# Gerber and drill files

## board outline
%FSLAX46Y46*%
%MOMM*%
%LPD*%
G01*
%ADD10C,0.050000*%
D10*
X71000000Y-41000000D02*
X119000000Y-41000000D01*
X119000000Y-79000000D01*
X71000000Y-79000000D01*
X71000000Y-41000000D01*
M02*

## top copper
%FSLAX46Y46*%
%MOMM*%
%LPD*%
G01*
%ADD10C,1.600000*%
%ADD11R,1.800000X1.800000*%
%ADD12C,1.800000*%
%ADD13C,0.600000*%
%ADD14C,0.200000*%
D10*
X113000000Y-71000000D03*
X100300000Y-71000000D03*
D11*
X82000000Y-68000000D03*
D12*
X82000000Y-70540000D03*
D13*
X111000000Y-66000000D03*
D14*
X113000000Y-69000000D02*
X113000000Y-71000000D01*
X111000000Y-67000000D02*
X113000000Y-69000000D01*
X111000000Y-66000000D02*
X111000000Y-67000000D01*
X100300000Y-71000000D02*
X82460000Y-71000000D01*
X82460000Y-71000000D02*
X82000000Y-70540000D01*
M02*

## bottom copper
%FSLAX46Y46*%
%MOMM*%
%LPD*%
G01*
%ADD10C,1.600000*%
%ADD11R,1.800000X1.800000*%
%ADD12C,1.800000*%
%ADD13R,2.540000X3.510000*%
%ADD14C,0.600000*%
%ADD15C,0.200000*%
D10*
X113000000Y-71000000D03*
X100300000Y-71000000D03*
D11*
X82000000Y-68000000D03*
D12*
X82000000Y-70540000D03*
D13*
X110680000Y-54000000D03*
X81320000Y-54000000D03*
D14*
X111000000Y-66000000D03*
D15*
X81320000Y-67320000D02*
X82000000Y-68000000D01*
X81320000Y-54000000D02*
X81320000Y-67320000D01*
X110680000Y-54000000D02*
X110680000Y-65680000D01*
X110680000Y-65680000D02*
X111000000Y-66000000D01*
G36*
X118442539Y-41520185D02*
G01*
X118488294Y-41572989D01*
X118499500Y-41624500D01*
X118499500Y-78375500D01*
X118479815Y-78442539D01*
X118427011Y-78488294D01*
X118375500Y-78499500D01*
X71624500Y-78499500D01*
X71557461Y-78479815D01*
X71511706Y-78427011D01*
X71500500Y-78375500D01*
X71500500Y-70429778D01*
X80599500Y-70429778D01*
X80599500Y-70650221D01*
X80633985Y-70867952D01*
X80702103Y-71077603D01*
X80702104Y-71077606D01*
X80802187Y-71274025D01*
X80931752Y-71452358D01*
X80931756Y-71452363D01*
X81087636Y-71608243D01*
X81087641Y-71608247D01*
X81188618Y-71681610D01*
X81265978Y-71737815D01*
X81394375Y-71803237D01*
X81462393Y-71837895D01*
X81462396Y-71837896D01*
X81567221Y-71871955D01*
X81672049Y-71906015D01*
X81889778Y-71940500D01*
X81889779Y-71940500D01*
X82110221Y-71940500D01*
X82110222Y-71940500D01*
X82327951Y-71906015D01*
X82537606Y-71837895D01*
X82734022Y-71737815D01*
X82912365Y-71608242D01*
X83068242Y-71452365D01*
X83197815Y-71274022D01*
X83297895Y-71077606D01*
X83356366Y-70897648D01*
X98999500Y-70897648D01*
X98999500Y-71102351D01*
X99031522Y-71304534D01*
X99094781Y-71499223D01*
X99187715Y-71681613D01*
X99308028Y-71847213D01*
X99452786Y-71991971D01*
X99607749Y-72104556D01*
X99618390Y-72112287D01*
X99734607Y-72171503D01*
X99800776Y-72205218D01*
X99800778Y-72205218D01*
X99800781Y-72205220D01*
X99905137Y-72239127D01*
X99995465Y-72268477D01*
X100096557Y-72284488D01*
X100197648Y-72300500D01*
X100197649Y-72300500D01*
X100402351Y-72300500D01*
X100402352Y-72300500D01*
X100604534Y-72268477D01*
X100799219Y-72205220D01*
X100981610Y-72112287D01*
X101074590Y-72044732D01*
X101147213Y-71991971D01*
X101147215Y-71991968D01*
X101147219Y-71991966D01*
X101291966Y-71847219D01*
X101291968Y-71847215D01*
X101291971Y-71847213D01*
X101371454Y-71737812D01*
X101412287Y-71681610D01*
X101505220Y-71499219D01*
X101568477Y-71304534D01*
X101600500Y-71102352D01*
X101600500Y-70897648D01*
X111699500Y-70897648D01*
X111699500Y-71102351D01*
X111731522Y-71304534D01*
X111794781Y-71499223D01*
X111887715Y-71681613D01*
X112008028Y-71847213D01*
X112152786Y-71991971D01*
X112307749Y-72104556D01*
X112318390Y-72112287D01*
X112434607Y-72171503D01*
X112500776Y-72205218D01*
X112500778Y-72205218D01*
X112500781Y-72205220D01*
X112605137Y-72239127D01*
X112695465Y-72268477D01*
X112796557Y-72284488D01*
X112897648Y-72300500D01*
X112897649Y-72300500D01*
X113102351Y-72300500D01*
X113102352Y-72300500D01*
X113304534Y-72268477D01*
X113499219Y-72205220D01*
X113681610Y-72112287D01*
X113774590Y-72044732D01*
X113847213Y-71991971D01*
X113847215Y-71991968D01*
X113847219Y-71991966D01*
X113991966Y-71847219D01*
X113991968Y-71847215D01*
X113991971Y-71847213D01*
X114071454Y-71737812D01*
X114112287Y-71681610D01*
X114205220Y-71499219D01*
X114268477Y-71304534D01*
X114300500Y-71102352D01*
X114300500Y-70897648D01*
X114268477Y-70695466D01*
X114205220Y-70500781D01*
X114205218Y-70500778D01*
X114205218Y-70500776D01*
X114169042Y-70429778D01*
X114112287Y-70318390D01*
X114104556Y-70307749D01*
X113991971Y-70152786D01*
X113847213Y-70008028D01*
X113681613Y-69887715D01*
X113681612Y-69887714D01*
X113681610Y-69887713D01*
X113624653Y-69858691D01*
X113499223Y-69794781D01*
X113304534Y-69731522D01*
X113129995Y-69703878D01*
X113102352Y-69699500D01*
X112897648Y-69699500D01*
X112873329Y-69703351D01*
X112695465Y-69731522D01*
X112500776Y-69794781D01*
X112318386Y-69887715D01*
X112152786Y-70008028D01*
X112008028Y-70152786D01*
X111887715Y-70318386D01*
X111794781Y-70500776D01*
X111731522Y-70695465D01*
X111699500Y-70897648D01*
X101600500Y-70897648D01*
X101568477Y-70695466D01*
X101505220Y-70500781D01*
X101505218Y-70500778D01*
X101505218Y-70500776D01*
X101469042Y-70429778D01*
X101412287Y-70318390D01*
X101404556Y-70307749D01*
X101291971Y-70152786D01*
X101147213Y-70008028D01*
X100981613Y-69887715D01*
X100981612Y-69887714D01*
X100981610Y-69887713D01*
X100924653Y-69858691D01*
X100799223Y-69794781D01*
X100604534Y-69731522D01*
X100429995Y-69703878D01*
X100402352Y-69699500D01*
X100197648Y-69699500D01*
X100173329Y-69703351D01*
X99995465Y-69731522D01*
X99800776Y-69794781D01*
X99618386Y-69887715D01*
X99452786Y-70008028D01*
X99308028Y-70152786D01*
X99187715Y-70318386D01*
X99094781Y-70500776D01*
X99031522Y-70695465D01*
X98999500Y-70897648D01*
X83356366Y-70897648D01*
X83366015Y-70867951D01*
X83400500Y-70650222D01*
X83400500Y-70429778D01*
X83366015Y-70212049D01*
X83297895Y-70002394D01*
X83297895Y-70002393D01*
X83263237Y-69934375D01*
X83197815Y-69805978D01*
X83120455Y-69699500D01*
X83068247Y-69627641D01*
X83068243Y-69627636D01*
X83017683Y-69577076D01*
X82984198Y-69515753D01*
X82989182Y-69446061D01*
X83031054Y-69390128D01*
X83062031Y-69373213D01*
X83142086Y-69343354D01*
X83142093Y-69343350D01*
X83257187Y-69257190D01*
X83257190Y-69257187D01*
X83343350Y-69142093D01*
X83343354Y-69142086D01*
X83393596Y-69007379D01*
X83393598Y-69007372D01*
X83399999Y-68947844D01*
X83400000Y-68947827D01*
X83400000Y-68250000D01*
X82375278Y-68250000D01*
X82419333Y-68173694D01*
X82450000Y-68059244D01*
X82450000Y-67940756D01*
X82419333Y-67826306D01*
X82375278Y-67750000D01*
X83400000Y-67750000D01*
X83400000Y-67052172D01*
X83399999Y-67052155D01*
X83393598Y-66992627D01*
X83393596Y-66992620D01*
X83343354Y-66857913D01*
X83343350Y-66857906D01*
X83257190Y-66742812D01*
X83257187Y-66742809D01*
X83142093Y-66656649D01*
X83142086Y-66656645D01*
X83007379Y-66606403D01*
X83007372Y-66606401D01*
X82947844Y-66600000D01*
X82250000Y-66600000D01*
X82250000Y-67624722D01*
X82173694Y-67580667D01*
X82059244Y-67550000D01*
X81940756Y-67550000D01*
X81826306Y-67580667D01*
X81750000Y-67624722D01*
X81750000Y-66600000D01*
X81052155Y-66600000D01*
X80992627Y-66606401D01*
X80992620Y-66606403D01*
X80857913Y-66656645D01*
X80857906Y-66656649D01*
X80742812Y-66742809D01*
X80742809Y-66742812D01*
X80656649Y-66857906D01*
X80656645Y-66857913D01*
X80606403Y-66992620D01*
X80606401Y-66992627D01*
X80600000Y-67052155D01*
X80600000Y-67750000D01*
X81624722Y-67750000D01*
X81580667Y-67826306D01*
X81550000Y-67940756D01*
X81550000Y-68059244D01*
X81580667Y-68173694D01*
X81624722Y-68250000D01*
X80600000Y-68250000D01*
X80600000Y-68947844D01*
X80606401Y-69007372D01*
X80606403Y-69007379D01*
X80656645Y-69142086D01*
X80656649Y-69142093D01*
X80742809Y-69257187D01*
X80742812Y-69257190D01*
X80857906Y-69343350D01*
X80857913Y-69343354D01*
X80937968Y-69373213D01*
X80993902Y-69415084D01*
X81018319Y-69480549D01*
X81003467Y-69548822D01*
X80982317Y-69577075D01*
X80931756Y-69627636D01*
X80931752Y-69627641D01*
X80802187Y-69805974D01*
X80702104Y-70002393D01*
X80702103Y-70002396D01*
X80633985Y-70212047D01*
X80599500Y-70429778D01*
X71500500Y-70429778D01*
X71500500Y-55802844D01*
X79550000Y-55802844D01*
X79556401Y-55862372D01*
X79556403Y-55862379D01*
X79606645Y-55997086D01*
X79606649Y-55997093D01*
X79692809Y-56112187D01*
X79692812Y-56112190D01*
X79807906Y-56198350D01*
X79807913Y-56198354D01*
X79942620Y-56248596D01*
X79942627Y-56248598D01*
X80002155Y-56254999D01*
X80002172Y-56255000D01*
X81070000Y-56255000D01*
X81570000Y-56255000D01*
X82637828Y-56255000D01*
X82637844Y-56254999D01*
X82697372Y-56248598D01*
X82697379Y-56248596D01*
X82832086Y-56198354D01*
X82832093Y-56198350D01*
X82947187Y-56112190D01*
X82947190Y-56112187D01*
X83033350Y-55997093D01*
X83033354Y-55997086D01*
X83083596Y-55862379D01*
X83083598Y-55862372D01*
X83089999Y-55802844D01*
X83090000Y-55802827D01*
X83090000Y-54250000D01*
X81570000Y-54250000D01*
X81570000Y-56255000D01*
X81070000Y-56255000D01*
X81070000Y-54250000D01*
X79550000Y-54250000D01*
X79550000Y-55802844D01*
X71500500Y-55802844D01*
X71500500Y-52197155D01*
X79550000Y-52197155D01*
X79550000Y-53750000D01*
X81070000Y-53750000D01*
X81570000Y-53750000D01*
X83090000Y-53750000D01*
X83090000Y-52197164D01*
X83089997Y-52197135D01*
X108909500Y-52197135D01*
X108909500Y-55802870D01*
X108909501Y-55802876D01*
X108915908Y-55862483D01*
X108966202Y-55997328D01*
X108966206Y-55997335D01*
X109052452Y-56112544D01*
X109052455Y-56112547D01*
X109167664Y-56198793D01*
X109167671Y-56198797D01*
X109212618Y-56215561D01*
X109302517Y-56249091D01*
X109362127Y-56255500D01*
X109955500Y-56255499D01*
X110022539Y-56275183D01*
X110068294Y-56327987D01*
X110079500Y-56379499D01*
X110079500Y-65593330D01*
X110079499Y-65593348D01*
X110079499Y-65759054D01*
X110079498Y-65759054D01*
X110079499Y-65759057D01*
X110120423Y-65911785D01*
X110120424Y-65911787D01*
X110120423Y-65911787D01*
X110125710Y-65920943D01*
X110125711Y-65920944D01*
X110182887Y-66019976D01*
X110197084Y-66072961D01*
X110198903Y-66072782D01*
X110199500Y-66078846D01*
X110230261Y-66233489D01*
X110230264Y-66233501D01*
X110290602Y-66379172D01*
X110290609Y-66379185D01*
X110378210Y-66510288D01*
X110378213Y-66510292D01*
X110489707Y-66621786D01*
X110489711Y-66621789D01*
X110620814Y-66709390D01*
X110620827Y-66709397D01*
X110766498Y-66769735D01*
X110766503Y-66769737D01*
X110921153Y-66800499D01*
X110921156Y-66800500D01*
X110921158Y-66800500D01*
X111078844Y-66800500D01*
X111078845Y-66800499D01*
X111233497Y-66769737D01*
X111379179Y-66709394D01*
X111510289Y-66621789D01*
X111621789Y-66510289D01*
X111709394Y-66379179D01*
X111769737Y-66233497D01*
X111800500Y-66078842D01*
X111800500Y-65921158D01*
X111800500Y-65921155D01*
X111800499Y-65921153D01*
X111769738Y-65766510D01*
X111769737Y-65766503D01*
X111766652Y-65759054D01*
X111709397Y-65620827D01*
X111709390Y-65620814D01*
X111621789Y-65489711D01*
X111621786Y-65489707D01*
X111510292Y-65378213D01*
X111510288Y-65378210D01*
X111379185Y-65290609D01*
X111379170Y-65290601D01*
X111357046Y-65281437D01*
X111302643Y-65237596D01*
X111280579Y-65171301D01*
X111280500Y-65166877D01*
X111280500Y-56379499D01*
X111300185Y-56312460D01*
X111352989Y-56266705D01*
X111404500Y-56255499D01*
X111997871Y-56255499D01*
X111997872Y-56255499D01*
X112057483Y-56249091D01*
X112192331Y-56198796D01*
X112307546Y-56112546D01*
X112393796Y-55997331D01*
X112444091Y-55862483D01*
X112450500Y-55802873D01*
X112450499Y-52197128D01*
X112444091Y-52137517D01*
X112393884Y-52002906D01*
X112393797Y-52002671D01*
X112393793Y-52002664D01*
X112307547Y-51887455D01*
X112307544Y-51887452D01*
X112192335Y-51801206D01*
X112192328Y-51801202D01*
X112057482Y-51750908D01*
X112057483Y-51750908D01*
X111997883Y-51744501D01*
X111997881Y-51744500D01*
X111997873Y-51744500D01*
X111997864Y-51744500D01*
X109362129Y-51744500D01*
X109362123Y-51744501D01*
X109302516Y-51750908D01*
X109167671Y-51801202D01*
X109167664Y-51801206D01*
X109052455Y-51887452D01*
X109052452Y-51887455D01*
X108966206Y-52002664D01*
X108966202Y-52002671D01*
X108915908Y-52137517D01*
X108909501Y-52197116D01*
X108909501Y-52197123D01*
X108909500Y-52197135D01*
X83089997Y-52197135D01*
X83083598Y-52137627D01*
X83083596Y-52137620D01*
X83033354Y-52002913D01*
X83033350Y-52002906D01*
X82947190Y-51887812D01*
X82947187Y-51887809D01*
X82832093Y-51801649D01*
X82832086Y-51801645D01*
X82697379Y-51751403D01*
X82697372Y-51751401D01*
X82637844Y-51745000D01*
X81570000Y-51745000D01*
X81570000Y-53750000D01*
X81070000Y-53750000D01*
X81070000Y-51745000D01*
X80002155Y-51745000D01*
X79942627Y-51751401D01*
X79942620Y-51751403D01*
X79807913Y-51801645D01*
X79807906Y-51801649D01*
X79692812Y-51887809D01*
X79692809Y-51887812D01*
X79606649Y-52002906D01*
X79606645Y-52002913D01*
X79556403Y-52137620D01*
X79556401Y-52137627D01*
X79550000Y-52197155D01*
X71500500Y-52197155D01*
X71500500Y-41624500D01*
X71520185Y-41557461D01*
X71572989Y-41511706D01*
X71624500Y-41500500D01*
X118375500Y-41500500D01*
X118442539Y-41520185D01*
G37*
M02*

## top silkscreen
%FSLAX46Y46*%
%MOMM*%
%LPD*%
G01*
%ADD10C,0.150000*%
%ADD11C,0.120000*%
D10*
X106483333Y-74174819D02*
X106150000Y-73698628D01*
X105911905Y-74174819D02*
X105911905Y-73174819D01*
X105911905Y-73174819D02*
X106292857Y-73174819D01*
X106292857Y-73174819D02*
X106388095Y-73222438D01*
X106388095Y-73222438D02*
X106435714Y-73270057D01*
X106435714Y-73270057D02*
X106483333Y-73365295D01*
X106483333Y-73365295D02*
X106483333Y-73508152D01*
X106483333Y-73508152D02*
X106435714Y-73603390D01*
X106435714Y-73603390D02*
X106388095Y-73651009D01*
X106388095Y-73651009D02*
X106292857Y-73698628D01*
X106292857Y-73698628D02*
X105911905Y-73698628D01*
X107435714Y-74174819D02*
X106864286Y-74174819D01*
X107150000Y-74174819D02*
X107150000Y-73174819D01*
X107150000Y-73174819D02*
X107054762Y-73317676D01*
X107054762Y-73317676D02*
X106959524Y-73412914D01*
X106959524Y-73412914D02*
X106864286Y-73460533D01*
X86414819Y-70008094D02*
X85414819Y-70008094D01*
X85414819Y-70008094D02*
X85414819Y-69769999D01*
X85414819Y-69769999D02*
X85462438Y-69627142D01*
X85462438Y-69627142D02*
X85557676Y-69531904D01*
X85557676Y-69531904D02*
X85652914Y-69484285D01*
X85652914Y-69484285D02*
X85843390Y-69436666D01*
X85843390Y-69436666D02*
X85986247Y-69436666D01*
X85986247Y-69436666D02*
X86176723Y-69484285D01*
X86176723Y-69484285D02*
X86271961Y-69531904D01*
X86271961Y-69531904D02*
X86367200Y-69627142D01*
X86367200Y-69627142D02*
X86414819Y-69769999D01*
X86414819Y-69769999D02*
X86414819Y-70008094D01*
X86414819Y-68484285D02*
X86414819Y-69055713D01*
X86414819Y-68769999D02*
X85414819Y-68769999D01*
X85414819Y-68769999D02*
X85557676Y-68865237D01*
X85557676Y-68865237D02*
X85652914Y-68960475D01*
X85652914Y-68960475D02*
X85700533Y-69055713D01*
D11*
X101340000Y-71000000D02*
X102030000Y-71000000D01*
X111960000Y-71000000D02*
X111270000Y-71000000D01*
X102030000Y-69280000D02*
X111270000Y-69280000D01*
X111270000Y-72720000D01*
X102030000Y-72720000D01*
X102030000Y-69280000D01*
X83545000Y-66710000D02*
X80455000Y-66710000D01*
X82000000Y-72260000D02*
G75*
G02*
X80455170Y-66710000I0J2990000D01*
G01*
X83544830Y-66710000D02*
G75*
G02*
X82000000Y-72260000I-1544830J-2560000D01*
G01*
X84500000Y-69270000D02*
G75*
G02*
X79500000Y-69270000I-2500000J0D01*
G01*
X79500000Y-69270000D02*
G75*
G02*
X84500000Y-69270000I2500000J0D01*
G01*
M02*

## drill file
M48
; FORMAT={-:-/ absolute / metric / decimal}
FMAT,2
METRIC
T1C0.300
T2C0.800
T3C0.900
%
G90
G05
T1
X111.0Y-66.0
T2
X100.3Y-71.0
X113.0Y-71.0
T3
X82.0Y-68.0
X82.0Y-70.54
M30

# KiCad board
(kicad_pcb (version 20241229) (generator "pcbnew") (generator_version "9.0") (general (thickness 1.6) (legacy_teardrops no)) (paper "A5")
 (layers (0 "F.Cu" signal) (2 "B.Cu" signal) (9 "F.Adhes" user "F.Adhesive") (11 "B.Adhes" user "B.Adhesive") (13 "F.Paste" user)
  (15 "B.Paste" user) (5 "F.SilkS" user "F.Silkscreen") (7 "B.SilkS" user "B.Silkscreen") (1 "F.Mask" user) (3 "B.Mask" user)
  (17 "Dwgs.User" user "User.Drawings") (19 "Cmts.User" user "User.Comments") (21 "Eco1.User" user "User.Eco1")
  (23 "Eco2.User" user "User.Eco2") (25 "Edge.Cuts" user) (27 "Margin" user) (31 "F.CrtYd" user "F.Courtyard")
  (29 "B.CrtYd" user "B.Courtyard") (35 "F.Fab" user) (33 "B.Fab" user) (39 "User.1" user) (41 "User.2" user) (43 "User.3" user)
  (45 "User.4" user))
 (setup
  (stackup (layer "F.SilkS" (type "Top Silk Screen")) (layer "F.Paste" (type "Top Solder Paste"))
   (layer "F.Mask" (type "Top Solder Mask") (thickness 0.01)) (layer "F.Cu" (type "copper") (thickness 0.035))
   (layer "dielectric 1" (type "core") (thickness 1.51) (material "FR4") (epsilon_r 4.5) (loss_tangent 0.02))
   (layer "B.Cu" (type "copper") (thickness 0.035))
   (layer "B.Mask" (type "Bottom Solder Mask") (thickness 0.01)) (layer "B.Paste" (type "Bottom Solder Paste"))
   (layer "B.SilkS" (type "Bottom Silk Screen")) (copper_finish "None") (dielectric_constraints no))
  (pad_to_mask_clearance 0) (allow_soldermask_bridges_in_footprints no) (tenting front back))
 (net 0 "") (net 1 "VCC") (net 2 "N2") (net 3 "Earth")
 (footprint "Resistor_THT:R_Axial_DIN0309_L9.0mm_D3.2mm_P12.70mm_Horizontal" (layer "F.Cu") (at 113 71 180)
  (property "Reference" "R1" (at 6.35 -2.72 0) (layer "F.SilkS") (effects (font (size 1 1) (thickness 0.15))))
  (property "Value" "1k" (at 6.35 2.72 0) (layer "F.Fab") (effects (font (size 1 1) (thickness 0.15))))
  (fp_line (start 11.66 0) (end 10.97 0) (stroke (width 0.12) (type solid)) (layer "F.SilkS"))
  (fp_line (start 1.04 0) (end 1.73 0) (stroke (width 0.12) (type solid)) (layer "F.SilkS"))
  (fp_rect (start 1.73 -1.72) (end 10.97 1.72) (stroke (width 0.12) (type solid)) (fill no) (layer "F.SilkS"))
  (pad "1" thru_hole circle (at 0 0 180) (size 1.6 1.6) (drill 0.8) (layers "*.Cu" "*.Mask") (remove_unused_layers no) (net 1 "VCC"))
  (pad "2" thru_hole circle (at 12.7 0 180) (size 1.6 1.6) (drill 0.8) (layers "*.Cu" "*.Mask") (remove_unused_layers no) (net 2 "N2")))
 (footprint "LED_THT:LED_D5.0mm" (layer "F.Cu") (at 82 68 -90)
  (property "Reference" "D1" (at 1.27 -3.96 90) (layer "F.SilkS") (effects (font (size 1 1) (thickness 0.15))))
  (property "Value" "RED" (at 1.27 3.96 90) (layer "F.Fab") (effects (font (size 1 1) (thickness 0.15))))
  (fp_line (start -1.29 -1.545) (end -1.29 1.545) (stroke (width 0.12) (type solid)) (layer "F.SilkS"))
  (fp_arc (start 4.26 0) (mid 2.071779 2.880495) (end -1.29 1.54483) (stroke (width 0.12) (type solid)) (layer "F.SilkS"))
  (fp_arc (start -1.29 -1.54483) (mid 2.071779 -2.880495) (end 4.26 0) (stroke (width 0.12) (type solid)) (layer "F.SilkS"))
  (fp_circle (center 1.27 0) (end 3.77 0) (stroke (width 0.12) (type solid)) (fill no) (layer "F.SilkS"))
  (pad "1" thru_hole rect (at 0 0 270) (size 1.8 1.8) (drill 0.9) (layers "*.Cu" "*.Mask") (remove_unused_layers no) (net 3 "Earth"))
  (pad "2" thru_hole circle (at 2.54 0 270) (size 1.8 1.8) (drill 0.9) (layers "*.Cu" "*.Mask") (remove_unused_layers no) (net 2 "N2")))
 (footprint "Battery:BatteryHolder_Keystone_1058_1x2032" (layer "B.Cu") (at 96 54 180)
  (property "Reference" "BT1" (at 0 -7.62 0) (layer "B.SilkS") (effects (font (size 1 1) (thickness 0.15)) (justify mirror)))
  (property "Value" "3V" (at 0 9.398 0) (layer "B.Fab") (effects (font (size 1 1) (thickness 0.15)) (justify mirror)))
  (pad "1" smd rect (at -14.68 0 180) (size 2.54 3.51) (layers "B.Cu" "B.Mask" "B.Paste") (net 1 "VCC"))
  (pad "2" smd rect (at 14.68 0 180) (size 2.54 3.51) (layers "B.Cu" "B.Mask" "B.Paste") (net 3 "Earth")))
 (gr_rect (start 71 41) (end 119 79) (stroke (width 0.05) (type default)) (fill no) (layer "Edge.Cuts"))
 (segment (start 81.32 67.32) (end 82 68) (width 0.2) (layer "B.Cu") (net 3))
 (segment (start 81.32 54) (end 81.32 67.32) (width 0.2) (layer "B.Cu") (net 3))
 (segment (start 113 69) (end 113 71) (width 0.2) (layer "F.Cu") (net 1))
 (segment (start 111 67) (end 113 69) (width 0.2) (layer "F.Cu") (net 1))
 (segment (start 111 66) (end 111 67) (width 0.2) (layer "F.Cu") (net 1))
 (via (at 111 66) (size 0.6) (drill 0.3) (layers "F.Cu" "B.Cu") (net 1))
 (segment (start 110.68 54) (end 110.68 65.68) (width 0.2) (layer "B.Cu") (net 1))
 (segment (start 110.68 65.68) (end 111 66) (width 0.2) (layer "B.Cu") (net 1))
 (segment (start 100.3 71) (end 82.46 71) (width 0.2) (layer "F.Cu") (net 2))
 (segment (start 82.46 71) (end 82 70.54) (width 0.2) (layer "F.Cu") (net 2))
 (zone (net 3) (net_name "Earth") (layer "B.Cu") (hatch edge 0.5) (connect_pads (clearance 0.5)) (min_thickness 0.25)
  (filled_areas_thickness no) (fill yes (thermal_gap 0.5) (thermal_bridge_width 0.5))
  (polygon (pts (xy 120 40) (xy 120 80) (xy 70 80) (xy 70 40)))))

